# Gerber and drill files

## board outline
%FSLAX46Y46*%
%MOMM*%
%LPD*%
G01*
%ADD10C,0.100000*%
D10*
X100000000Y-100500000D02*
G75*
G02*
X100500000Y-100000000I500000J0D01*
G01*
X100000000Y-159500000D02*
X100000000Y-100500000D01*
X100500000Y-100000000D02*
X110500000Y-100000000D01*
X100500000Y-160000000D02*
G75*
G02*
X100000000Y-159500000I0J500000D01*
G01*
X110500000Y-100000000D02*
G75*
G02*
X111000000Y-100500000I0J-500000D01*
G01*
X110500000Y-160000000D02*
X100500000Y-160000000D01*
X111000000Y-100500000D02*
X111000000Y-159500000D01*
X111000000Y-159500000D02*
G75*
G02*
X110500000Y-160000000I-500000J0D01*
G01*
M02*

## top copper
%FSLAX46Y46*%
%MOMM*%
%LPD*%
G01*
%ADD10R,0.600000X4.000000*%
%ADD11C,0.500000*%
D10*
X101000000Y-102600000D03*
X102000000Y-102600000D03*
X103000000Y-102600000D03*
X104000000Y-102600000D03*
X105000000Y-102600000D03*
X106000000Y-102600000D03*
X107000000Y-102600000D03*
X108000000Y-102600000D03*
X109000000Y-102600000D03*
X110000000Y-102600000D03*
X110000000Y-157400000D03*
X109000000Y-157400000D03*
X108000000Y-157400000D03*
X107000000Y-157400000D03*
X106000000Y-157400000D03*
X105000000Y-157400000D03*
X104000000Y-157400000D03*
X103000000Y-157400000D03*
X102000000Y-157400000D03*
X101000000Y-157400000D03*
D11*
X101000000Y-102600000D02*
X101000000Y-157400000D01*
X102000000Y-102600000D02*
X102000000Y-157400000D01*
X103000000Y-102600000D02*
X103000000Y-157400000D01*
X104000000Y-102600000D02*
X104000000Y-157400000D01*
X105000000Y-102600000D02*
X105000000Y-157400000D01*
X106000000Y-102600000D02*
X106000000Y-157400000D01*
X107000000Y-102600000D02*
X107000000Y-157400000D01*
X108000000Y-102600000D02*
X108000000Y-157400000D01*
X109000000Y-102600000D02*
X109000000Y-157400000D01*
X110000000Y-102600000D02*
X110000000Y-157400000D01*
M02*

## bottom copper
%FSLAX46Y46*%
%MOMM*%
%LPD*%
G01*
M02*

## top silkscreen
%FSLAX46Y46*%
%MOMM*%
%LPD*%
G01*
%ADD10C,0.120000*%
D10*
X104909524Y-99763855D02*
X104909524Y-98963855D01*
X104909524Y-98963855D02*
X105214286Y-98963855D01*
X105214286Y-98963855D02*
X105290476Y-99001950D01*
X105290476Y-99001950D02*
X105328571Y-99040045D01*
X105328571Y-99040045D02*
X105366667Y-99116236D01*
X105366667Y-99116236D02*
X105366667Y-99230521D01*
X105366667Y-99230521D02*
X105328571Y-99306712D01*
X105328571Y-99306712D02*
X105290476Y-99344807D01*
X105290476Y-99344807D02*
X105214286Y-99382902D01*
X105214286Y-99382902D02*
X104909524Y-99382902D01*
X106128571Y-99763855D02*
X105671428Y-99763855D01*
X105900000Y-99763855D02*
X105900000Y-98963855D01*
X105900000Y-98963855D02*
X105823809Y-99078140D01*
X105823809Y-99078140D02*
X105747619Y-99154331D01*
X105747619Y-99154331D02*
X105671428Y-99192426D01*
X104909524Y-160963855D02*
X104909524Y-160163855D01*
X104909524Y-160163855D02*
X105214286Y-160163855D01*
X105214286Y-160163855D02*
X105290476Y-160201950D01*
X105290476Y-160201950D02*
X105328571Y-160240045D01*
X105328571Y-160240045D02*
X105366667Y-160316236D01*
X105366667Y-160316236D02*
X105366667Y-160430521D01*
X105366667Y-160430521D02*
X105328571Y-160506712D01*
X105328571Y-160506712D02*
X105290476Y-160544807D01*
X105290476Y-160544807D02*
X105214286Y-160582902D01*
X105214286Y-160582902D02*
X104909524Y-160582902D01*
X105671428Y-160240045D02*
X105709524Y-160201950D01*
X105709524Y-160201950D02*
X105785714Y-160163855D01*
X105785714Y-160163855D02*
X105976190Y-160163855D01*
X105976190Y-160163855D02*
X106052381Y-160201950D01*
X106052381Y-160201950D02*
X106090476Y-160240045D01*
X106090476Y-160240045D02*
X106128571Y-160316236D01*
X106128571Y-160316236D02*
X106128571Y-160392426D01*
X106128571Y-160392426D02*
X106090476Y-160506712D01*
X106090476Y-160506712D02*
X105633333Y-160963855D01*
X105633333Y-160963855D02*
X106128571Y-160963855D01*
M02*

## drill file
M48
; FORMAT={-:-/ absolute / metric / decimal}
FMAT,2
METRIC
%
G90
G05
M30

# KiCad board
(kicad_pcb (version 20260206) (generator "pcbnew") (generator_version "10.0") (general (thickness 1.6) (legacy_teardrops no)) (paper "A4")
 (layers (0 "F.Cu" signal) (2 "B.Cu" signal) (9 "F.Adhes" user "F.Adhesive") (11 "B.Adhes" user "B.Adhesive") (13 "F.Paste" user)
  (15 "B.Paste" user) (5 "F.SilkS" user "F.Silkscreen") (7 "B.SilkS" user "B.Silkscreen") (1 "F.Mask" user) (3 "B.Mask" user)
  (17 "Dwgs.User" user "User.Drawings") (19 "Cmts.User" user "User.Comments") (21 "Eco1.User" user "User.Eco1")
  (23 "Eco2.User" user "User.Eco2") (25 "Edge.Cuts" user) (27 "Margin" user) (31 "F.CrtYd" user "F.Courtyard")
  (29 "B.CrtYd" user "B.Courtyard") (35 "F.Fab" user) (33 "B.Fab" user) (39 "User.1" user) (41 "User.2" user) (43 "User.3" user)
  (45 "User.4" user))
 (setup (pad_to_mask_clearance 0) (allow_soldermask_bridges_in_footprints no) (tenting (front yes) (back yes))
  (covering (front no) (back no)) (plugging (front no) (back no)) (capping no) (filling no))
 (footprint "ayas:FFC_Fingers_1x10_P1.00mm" (layer "F.Cu") (at 105.5 102.6)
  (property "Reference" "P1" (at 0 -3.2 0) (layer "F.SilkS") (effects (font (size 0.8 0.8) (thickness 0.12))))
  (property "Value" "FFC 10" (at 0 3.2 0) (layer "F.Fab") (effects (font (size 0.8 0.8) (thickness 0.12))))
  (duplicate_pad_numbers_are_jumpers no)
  (pad "1" smd rect (at -4.5 0) (size 0.6 4) (layers "F.Cu" "F.Mask") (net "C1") (solder_mask_margin 0))
  (pad "2" smd rect (at -3.5 0) (size 0.6 4) (layers "F.Cu" "F.Mask") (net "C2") (solder_mask_margin 0))
  (pad "3" smd rect (at -2.5 0) (size 0.6 4) (layers "F.Cu" "F.Mask") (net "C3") (solder_mask_margin 0))
  (pad "4" smd rect (at -1.5 0) (size 0.6 4) (layers "F.Cu" "F.Mask") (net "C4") (solder_mask_margin 0))
  (pad "5" smd rect (at -0.5 0) (size 0.6 4) (layers "F.Cu" "F.Mask") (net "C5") (solder_mask_margin 0))
  (pad "6" smd rect (at 0.5 0) (size 0.6 4) (layers "F.Cu" "F.Mask") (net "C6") (solder_mask_margin 0))
  (pad "7" smd rect (at 1.5 0) (size 0.6 4) (layers "F.Cu" "F.Mask") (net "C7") (solder_mask_margin 0))
  (pad "8" smd rect (at 2.5 0) (size 0.6 4) (layers "F.Cu" "F.Mask") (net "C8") (solder_mask_margin 0))
  (pad "9" smd rect (at 3.5 0) (size 0.6 4) (layers "F.Cu" "F.Mask") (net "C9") (solder_mask_margin 0))
  (pad "10" smd rect (at 4.5 0) (size 0.6 4) (layers "F.Cu" "F.Mask") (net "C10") (solder_mask_margin 0)))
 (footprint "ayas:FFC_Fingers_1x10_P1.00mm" (layer "F.Cu") (at 105.5 157.4 180)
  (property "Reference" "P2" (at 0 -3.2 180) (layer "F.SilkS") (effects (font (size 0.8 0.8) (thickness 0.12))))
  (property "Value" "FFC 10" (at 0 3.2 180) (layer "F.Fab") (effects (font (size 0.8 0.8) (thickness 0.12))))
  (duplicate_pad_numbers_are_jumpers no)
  (pad "1" smd rect (at -4.5 0 180) (size 0.6 4) (layers "F.Cu" "F.Mask") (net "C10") (solder_mask_margin 0))
  (pad "2" smd rect (at -3.5 0 180) (size 0.6 4) (layers "F.Cu" "F.Mask") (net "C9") (solder_mask_margin 0))
  (pad "3" smd rect (at -2.5 0 180) (size 0.6 4) (layers "F.Cu" "F.Mask") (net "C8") (solder_mask_margin 0))
  (pad "4" smd rect (at -1.5 0 180) (size 0.6 4) (layers "F.Cu" "F.Mask") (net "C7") (solder_mask_margin 0))
  (pad "5" smd rect (at -0.5 0 180) (size 0.6 4) (layers "F.Cu" "F.Mask") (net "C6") (solder_mask_margin 0))
  (pad "6" smd rect (at 0.5 0 180) (size 0.6 4) (layers "F.Cu" "F.Mask") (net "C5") (solder_mask_margin 0))
  (pad "7" smd rect (at 1.5 0 180) (size 0.6 4) (layers "F.Cu" "F.Mask") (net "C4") (solder_mask_margin 0))
  (pad "8" smd rect (at 2.5 0 180) (size 0.6 4) (layers "F.Cu" "F.Mask") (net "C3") (solder_mask_margin 0))
  (pad "9" smd rect (at 3.5 0 180) (size 0.6 4) (layers "F.Cu" "F.Mask") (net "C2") (solder_mask_margin 0))
  (pad "10" smd rect (at 4.5 0 180) (size 0.6 4) (layers "F.Cu" "F.Mask") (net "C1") (solder_mask_margin 0)))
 (gr_arc (start 100 100.5) (mid 100.146447 100.146447) (end 100.5 100) (stroke (width 0.1) (type default)) (layer "Edge.Cuts"))
 (gr_line (start 100 159.5) (end 100 100.5) (stroke (width 0.1) (type default)) (layer "Edge.Cuts"))
 (gr_line (start 100.5 100) (end 110.5 100) (stroke (width 0.1) (type default)) (layer "Edge.Cuts"))
 (gr_arc (start 100.5 160) (mid 100.146447 159.853553) (end 100 159.5) (stroke (width 0.1) (type default)) (layer "Edge.Cuts"))
 (gr_arc (start 110.5 100) (mid 110.853553 100.146447) (end 111 100.5) (stroke (width 0.1) (type default)) (layer "Edge.Cuts"))
 (gr_line (start 110.5 160) (end 100.5 160) (stroke (width 0.1) (type default)) (layer "Edge.Cuts"))
 (gr_line (start 111 100.5) (end 111 159.5) (stroke (width 0.1) (type default)) (layer "Edge.Cuts"))
 (gr_arc (start 111 159.5) (mid 110.853553 159.853553) (end 110.5 160) (stroke (width 0.1) (type default)) (layer "Edge.Cuts"))
 (segment (start 101 102.6) (end 101 157.4) (width 0.5) (layer "F.Cu") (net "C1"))
 (segment (start 102 102.6) (end 102 157.4) (width 0.5) (layer "F.Cu") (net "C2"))
 (segment (start 103 102.6) (end 103 157.4) (width 0.5) (layer "F.Cu") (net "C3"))
 (segment (start 104 102.6) (end 104 157.4) (width 0.5) (layer "F.Cu") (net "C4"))
 (segment (start 105 102.6) (end 105 157.4) (width 0.5) (layer "F.Cu") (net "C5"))
 (segment (start 106 102.6) (end 106 157.4) (width 0.5) (layer "F.Cu") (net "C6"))
 (segment (start 107 102.6) (end 107 157.4) (width 0.5) (layer "F.Cu") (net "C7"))
 (segment (start 108 102.6) (end 108 157.4) (width 0.5) (layer "F.Cu") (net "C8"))
 (segment (start 109 102.6) (end 109 157.4) (width 0.5) (layer "F.Cu") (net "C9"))
 (segment (start 110 102.6) (end 110 157.4) (width 0.5) (layer "F.Cu") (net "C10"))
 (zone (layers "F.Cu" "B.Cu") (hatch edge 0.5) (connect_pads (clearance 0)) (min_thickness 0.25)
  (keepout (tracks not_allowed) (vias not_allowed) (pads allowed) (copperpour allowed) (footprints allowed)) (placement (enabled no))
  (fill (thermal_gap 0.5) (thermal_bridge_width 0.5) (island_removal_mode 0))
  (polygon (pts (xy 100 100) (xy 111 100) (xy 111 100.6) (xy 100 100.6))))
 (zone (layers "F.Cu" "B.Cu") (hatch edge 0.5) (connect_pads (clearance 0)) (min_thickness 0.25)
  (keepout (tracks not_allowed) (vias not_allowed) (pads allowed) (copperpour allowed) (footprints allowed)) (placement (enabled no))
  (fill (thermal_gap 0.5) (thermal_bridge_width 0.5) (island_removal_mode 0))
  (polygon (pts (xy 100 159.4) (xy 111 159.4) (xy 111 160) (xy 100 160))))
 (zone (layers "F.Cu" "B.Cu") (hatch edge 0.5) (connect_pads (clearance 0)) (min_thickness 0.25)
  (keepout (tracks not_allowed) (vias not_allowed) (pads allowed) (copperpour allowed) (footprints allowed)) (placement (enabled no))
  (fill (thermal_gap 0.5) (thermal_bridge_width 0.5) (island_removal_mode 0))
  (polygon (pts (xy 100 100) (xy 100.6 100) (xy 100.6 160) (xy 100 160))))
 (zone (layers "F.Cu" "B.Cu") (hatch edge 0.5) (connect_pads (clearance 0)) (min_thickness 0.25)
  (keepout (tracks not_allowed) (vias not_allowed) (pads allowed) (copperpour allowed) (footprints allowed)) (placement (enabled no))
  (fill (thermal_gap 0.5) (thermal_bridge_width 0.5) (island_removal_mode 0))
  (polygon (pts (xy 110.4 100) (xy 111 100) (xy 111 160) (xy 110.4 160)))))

